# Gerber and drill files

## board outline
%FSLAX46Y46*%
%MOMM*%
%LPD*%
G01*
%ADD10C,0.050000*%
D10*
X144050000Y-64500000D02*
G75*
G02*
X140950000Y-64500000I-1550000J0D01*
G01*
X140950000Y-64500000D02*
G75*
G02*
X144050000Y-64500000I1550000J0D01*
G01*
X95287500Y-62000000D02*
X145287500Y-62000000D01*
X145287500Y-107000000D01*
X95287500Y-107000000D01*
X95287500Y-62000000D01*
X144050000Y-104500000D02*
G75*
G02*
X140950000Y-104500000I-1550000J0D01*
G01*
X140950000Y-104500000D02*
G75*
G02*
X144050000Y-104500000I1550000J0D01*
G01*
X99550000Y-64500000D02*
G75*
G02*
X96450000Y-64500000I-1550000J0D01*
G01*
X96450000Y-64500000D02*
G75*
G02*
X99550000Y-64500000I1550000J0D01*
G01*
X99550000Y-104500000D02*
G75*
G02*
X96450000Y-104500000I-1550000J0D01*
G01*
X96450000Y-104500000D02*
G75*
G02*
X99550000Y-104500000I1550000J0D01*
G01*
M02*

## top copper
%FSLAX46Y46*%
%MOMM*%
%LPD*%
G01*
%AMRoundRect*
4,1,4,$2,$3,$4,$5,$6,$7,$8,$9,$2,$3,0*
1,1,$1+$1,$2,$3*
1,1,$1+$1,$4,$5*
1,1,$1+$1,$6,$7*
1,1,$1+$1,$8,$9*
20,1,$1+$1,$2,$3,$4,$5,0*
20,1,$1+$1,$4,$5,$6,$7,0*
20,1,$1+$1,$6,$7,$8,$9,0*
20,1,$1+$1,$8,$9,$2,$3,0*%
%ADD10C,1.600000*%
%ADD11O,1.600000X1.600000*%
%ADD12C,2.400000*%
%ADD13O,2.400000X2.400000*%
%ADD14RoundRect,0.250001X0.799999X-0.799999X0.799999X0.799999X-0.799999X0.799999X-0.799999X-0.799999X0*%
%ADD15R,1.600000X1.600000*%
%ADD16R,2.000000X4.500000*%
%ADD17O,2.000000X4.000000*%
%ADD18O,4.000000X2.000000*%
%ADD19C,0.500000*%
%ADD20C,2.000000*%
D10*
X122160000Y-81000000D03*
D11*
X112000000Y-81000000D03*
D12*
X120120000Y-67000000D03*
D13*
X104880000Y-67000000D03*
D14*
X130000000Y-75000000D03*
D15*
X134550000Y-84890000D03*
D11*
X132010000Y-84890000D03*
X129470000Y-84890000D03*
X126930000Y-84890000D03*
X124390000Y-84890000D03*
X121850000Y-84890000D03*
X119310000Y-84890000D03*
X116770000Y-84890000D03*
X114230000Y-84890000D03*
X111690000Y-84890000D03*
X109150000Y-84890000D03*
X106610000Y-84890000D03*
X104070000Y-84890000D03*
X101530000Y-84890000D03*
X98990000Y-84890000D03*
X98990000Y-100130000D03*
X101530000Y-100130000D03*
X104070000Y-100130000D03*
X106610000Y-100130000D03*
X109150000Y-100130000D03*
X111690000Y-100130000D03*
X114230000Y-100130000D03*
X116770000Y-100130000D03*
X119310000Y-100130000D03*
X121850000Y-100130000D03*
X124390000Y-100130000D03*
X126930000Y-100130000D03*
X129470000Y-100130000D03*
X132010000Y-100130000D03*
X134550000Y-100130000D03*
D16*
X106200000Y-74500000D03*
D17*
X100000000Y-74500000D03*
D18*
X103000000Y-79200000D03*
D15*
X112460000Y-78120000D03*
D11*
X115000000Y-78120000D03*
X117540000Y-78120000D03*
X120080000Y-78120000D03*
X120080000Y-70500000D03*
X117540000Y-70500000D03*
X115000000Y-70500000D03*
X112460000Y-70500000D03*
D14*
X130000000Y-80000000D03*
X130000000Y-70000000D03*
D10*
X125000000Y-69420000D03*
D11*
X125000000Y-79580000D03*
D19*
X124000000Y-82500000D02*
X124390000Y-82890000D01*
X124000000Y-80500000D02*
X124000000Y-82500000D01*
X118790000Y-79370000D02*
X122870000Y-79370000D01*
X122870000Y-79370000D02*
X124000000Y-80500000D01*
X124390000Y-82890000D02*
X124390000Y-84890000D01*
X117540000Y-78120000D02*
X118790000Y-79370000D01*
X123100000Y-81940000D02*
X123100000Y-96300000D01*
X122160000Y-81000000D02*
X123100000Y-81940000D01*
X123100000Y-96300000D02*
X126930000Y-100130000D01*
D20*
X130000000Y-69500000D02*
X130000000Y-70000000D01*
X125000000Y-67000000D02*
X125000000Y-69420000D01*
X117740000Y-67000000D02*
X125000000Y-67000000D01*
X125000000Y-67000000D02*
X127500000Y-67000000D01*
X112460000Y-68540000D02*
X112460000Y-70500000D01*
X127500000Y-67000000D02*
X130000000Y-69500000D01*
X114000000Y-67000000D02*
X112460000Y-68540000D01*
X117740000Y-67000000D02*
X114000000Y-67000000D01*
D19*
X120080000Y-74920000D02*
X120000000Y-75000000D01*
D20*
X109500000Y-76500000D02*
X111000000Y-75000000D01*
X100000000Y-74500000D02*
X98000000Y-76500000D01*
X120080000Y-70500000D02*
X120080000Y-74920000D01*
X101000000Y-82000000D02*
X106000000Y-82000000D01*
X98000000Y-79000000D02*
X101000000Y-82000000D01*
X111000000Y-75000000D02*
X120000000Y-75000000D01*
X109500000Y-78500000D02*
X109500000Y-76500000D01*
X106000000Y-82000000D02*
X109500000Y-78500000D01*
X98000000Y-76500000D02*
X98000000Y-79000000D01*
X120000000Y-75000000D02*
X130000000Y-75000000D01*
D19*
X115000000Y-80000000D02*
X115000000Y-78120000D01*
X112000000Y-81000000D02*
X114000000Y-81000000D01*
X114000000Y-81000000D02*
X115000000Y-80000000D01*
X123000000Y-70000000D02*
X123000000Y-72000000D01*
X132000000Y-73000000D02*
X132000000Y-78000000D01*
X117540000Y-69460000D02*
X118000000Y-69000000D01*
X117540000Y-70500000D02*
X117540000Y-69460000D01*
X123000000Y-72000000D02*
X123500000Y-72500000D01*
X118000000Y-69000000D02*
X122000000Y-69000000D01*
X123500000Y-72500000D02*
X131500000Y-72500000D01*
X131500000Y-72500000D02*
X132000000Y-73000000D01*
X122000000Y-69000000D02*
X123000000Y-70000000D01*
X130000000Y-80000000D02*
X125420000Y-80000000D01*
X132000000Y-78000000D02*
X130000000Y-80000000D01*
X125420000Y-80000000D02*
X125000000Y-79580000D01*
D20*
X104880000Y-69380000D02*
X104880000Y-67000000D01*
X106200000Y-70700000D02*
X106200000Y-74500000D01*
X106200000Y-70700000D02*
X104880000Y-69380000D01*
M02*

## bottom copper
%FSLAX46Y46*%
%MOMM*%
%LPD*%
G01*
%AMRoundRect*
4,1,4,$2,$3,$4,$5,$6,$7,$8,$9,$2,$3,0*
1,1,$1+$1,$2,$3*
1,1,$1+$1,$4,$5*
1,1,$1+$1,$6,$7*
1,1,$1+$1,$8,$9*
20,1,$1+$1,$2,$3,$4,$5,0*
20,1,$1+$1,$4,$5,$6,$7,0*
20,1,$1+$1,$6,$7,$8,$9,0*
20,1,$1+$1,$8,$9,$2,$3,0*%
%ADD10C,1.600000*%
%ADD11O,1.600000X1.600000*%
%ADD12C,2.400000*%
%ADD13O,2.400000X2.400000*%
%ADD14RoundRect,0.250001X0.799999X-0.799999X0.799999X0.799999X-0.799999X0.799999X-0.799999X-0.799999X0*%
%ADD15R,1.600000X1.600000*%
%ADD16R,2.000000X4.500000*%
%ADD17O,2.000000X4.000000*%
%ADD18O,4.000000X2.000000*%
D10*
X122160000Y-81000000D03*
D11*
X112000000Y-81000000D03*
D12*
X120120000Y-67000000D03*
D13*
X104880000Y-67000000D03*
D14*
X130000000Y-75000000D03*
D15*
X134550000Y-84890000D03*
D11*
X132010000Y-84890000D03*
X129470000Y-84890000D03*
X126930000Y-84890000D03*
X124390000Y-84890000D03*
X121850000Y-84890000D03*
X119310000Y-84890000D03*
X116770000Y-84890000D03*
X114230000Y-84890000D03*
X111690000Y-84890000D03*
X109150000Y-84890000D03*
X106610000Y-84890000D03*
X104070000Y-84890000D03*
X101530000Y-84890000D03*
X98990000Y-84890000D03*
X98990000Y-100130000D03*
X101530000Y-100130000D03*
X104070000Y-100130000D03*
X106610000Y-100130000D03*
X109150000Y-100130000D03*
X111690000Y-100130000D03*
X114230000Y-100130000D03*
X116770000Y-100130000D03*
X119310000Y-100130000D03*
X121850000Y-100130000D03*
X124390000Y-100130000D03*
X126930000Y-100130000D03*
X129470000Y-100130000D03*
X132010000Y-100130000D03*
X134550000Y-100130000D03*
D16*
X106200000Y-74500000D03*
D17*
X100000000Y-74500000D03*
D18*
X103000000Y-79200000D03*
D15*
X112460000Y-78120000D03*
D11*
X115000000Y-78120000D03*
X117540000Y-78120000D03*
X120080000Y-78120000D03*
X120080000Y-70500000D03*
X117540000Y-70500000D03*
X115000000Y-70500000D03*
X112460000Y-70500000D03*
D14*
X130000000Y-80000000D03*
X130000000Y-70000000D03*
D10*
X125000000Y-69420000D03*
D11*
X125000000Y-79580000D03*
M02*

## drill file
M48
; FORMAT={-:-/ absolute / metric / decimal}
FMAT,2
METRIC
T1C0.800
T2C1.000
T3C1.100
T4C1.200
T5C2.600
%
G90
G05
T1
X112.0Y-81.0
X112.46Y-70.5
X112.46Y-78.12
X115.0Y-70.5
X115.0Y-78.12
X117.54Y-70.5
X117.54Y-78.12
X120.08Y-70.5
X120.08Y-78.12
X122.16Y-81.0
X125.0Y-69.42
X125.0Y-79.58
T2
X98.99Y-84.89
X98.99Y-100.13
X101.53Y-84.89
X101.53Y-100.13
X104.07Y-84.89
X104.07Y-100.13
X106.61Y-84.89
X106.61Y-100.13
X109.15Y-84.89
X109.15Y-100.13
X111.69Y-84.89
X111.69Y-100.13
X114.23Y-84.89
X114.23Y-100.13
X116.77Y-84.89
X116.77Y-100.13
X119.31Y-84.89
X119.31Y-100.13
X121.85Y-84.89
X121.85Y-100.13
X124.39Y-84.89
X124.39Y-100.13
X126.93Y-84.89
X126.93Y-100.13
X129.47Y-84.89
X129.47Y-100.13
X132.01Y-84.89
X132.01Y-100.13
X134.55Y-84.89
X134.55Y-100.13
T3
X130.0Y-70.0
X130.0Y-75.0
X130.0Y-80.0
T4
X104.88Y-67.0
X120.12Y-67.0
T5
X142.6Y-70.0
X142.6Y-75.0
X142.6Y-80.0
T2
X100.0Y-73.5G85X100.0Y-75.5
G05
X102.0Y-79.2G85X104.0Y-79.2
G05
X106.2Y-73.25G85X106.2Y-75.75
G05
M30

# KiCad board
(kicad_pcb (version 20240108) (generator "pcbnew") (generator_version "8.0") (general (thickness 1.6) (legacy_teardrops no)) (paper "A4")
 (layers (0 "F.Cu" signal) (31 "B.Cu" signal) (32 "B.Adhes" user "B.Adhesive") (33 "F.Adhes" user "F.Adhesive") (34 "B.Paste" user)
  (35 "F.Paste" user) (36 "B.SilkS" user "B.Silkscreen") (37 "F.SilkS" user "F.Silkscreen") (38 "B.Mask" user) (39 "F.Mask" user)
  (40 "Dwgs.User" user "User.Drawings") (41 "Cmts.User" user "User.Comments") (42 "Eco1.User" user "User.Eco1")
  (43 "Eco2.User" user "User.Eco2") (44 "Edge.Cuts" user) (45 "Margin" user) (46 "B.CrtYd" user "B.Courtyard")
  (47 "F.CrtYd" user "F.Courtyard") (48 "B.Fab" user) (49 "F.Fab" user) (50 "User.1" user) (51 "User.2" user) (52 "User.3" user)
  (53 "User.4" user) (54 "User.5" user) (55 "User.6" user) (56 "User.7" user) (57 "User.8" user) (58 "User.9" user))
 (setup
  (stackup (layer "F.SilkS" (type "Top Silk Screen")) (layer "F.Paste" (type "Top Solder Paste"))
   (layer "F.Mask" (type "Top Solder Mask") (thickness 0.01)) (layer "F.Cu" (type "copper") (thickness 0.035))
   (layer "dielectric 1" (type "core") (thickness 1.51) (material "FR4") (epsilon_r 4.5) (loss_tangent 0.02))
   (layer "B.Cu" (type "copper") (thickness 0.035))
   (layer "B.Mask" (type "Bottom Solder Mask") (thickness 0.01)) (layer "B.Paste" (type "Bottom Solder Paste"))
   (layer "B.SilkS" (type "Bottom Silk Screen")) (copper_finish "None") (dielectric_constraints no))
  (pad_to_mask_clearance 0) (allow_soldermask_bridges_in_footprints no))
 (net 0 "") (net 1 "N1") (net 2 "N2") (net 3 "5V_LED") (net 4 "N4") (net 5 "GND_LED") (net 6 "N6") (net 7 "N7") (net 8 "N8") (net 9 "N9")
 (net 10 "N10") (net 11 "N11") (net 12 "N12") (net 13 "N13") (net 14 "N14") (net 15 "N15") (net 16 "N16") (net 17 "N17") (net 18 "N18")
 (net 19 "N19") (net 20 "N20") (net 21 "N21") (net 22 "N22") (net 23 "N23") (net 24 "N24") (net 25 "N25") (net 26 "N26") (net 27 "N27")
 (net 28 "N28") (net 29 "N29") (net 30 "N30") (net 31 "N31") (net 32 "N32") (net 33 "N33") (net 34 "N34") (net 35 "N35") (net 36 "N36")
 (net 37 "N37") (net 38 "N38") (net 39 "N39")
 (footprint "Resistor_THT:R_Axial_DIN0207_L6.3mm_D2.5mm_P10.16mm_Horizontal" (layer "F.Cu") (at 122.16 81 180)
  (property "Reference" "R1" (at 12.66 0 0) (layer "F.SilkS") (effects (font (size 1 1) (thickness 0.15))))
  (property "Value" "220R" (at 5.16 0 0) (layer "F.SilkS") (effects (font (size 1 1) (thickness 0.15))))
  (pad "1" thru_hole circle (at 0 0 180) (size 1.6 1.6) (drill 0.8) (layers "*.Cu" "*.Mask") (remove_unused_layers no) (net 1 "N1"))
  (pad "2" thru_hole oval (at 10.16 0 180) (size 1.6 1.6) (drill 0.8) (layers "*.Cu" "*.Mask") (remove_unused_layers no) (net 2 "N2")))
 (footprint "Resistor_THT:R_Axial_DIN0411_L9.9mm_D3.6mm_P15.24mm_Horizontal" (layer "F.Cu") (at 120.12 67 180)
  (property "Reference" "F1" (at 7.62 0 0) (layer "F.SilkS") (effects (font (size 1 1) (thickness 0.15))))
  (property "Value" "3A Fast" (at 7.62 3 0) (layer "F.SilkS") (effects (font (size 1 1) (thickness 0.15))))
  (pad "1" thru_hole circle (at 0 0 180) (size 2.4 2.4) (drill 1.2) (layers "*.Cu" "*.Mask") (remove_unused_layers no) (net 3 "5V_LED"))
  (pad "2" thru_hole oval (at 15.24 0 180) (size 2.4 2.4) (drill 1.2) (layers "*.Cu" "*.Mask") (remove_unused_layers no) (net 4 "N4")))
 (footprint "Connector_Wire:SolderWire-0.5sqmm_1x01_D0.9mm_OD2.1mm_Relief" (layer "F.Cu") (at 130 75 90)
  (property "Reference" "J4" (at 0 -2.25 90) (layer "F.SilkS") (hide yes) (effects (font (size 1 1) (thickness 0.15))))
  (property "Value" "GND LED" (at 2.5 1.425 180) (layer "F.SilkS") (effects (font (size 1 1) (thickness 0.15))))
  (pad "" np_thru_hole circle (at 0 12.6 90) (size 2.6 2.6) (drill 2.6) (layers "*.Cu" "*.Mask"))
  (pad "1" thru_hole roundrect (at 0 0 90) (size 2.1 2.1) (drill 1.1) (layers "*.Cu" "*.Mask") (remove_unused_layers no)
   (roundrect_rratio 0.119048) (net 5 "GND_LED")))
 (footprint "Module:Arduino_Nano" (layer "F.Cu") (at 134.55 84.89 -90)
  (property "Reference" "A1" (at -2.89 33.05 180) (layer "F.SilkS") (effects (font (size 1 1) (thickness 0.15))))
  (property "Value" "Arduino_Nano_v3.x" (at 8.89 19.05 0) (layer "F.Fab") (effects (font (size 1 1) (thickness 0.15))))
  (pad "1" thru_hole rect (at 0 0 270) (size 1.6 1.6) (drill 1) (layers "*.Cu" "*.Mask") (remove_unused_layers no) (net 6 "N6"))
  (pad "2" thru_hole oval (at 0 2.54 270) (size 1.6 1.6) (drill 1) (layers "*.Cu" "*.Mask") (remove_unused_layers no) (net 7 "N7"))
  (pad "3" thru_hole oval (at 0 5.08 270) (size 1.6 1.6) (drill 1) (layers "*.Cu" "*.Mask") (remove_unused_layers no) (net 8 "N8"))
  (pad "4" thru_hole oval (at 0 7.62 270) (size 1.6 1.6) (drill 1) (layers "*.Cu" "*.Mask") (remove_unused_layers no) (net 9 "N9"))
  (pad "5" thru_hole oval (at 0 10.16 270) (size 1.6 1.6) (drill 1) (layers "*.Cu" "*.Mask") (remove_unused_layers no) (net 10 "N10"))
  (pad "6" thru_hole oval (at 0 12.7 270) (size 1.6 1.6) (drill 1) (layers "*.Cu" "*.Mask") (remove_unused_layers no) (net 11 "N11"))
  (pad "7" thru_hole oval (at 0 15.24 270) (size 1.6 1.6) (drill 1) (layers "*.Cu" "*.Mask") (remove_unused_layers no) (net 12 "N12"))
  (pad "8" thru_hole oval (at 0 17.78 270) (size 1.6 1.6) (drill 1) (layers "*.Cu" "*.Mask") (remove_unused_layers no) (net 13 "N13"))
  (pad "9" thru_hole oval (at 0 20.32 270) (size 1.6 1.6) (drill 1) (layers "*.Cu" "*.Mask") (remove_unused_layers no) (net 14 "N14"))
  (pad "10" thru_hole oval (at 0 22.86 270) (size 1.6 1.6) (drill 1) (layers "*.Cu" "*.Mask") (remove_unused_layers no) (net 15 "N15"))
  (pad "11" thru_hole oval (at 0 25.4 270) (size 1.6 1.6) (drill 1) (layers "*.Cu" "*.Mask") (remove_unused_layers no) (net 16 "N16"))
  (pad "12" thru_hole oval (at 0 27.94 270) (size 1.6 1.6) (drill 1) (layers "*.Cu" "*.Mask") (remove_unused_layers no) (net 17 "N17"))
  (pad "13" thru_hole oval (at 0 30.48 270) (size 1.6 1.6) (drill 1) (layers "*.Cu" "*.Mask") (remove_unused_layers no) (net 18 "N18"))
  (pad "14" thru_hole oval (at 0 33.02 270) (size 1.6 1.6) (drill 1) (layers "*.Cu" "*.Mask") (remove_unused_layers no) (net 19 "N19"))
  (pad "15" thru_hole oval (at 0 35.56 270) (size 1.6 1.6) (drill 1) (layers "*.Cu" "*.Mask") (remove_unused_layers no) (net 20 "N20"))
  (pad "16" thru_hole oval (at 15.24 35.56 270) (size 1.6 1.6) (drill 1) (layers "*.Cu" "*.Mask") (remove_unused_layers no) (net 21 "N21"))
  (pad "17" thru_hole oval (at 15.24 33.02 270) (size 1.6 1.6) (drill 1) (layers "*.Cu" "*.Mask") (remove_unused_layers no) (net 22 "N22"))
  (pad "18" thru_hole oval (at 15.24 30.48 270) (size 1.6 1.6) (drill 1) (layers "*.Cu" "*.Mask") (remove_unused_layers no) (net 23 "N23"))
  (pad "19" thru_hole oval (at 15.24 27.94 270) (size 1.6 1.6) (drill 1) (layers "*.Cu" "*.Mask") (remove_unused_layers no) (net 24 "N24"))
  (pad "20" thru_hole oval (at 15.24 25.4 270) (size 1.6 1.6) (drill 1) (layers "*.Cu" "*.Mask") (remove_unused_layers no) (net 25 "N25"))
  (pad "21" thru_hole oval (at 15.24 22.86 270) (size 1.6 1.6) (drill 1) (layers "*.Cu" "*.Mask") (remove_unused_layers no) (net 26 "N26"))
  (pad "22" thru_hole oval (at 15.24 20.32 270) (size 1.6 1.6) (drill 1) (layers "*.Cu" "*.Mask") (remove_unused_layers no) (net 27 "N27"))
  (pad "23" thru_hole oval (at 15.24 17.78 270) (size 1.6 1.6) (drill 1) (layers "*.Cu" "*.Mask") (remove_unused_layers no) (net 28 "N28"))
  (pad "24" thru_hole oval (at 15.24 15.24 270) (size 1.6 1.6) (drill 1) (layers "*.Cu" "*.Mask") (remove_unused_layers no) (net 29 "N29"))
  (pad "25" thru_hole oval (at 15.24 12.7 270) (size 1.6 1.6) (drill 1) (layers "*.Cu" "*.Mask") (remove_unused_layers no) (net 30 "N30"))
  (pad "26" thru_hole oval (at 15.24 10.16 270) (size 1.6 1.6) (drill 1) (layers "*.Cu" "*.Mask") (remove_unused_layers no) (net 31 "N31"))
  (pad "27" thru_hole oval (at 15.24 7.62 270) (size 1.6 1.6) (drill 1) (layers "*.Cu" "*.Mask") (remove_unused_layers no) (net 1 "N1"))
  (pad "28" thru_hole oval (at 15.24 5.08 270) (size 1.6 1.6) (drill 1) (layers "*.Cu" "*.Mask") (remove_unused_layers no) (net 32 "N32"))
  (pad "29" thru_hole oval (at 15.24 2.54 270) (size 1.6 1.6) (drill 1) (layers "*.Cu" "*.Mask") (remove_unused_layers no) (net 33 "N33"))
  (pad "30" thru_hole oval (at 15.24 0 270) (size 1.6 1.6) (drill 1) (layers "*.Cu" "*.Mask") (remove_unused_layers no) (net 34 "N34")))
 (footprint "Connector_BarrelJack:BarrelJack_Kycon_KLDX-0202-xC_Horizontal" (layer "F.Cu") (at 106.2 74.5)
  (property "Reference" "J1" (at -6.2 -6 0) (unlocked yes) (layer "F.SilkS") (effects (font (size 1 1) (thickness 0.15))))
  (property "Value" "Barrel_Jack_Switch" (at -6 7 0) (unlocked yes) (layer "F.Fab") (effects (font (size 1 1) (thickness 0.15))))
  (pad "1" thru_hole rect (at 0 0) (size 2 4.5) (drill oval 1 3.5) (layers "*.Cu" "*.Mask") (remove_unused_layers no) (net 4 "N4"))
  (pad "2" thru_hole oval (at -6.2 0) (size 2 4) (drill oval 1 3) (layers "*.Cu" "*.Mask") (remove_unused_layers no) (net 5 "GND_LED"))
  (pad "3" thru_hole oval (at -3.2 4.7 90) (size 2 4) (drill oval 1 3) (layers "*.Cu" "*.Mask") (remove_unused_layers no) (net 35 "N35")))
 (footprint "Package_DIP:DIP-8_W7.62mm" (layer "F.Cu") (at 112.46 78.12 90)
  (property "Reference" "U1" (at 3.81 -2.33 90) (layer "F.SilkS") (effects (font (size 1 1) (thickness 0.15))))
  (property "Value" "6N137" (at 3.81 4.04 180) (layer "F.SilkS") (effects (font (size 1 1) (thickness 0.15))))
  (pad "1" thru_hole rect (at 0 0 90) (size 1.6 1.6) (drill 0.8) (layers "*.Cu" "*.Mask") (remove_unused_layers no) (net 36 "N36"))
  (pad "2" thru_hole oval (at 0 2.54 90) (size 1.6 1.6) (drill 0.8) (layers "*.Cu" "*.Mask") (remove_unused_layers no) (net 2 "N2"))
  (pad "3" thru_hole oval (at 0 5.08 90) (size 1.6 1.6) (drill 0.8) (layers "*.Cu" "*.Mask") (remove_unused_layers no) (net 10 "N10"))
  (pad "4" thru_hole oval (at 0 7.62 90) (size 1.6 1.6) (drill 0.8) (layers "*.Cu" "*.Mask") (remove_unused_layers no) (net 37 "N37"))
  (pad "5" thru_hole oval (at 7.62 7.62 90) (size 1.6 1.6) (drill 0.8) (layers "*.Cu" "*.Mask") (remove_unused_layers no) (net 5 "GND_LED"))
  (pad "6" thru_hole oval (at 7.62 5.08 90) (size 1.6 1.6) (drill 0.8) (layers "*.Cu" "*.Mask") (remove_unused_layers no) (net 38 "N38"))
  (pad "7" thru_hole oval (at 7.62 2.54 90) (size 1.6 1.6) (drill 0.8) (layers "*.Cu" "*.Mask") (remove_unused_layers no) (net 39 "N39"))
  (pad "8" thru_hole oval (at 7.62 0 90) (size 1.6 1.6) (drill 0.8) (layers "*.Cu" "*.Mask") (remove_unused_layers no) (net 3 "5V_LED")))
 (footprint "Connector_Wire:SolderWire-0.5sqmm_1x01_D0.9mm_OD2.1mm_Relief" (layer "F.Cu") (at 130 80 90)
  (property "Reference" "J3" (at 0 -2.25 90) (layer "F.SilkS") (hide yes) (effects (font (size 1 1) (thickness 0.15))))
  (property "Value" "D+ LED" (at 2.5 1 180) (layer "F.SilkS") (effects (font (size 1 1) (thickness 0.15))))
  (pad "" np_thru_hole circle (at 0 12.6 90) (size 2.6 2.6) (drill 2.6) (layers "*.Cu" "*.Mask"))
  (pad "1" thru_hole roundrect (at 0 0 90) (size 2.1 2.1) (drill 1.1) (layers "*.Cu" "*.Mask") (remove_unused_layers no)
   (roundrect_rratio 0.119048) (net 38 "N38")))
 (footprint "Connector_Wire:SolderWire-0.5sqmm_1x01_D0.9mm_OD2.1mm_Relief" (layer "F.Cu") (at 130 70 90)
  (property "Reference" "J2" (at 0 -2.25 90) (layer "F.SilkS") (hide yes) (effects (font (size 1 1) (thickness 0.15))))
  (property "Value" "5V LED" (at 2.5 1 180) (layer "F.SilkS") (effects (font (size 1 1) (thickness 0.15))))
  (pad "" np_thru_hole circle (at 0 12.6 90) (size 2.6 2.6) (drill 2.6) (layers "*.Cu" "*.Mask"))
  (pad "1" thru_hole roundrect (at 0 0 90) (size 2.1 2.1) (drill 1.1) (layers "*.Cu" "*.Mask") (remove_unused_layers no)
   (roundrect_rratio 0.119048) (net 3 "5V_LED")))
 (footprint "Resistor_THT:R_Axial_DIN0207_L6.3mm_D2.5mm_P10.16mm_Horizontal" (layer "F.Cu") (at 125 69.42 -90)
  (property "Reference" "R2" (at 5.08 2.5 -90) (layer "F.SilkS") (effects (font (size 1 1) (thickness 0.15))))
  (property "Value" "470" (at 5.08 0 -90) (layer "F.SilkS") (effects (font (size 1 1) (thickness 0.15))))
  (pad "1" thru_hole circle (at 0 0 270) (size 1.6 1.6) (drill 0.8) (layers "*.Cu" "*.Mask") (remove_unused_layers no) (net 3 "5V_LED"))
  (pad "2" thru_hole oval (at 10.16 0 270) (size 1.6 1.6) (drill 0.8) (layers "*.Cu" "*.Mask") (remove_unused_layers no) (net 38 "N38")))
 (gr_circle (center 142.5 64.5) (end 144.05 64.5) (stroke (width 0.05) (type default)) (fill none) (layer "Edge.Cuts"))
 (gr_rect (start 95.2875 62) (end 145.2875 107) (stroke (width 0.05) (type default)) (fill none) (layer "Edge.Cuts"))
 (gr_circle (center 142.5 104.5) (end 144.05 104.5) (stroke (width 0.05) (type default)) (fill none) (layer "Edge.Cuts"))
 (gr_circle (center 98 64.5) (end 99.55 64.5) (stroke (width 0.05) (type default)) (fill none) (layer "Edge.Cuts"))
 (gr_circle (center 98 104.5) (end 99.55 104.5) (stroke (width 0.05) (type default)) (fill none) (layer "Edge.Cuts"))
 (segment (start 124 82.5) (end 124.39 82.89) (width 0.5) (layer "F.Cu") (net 10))
 (segment (start 124 80.5) (end 124 82.5) (width 0.5) (layer "F.Cu") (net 10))
 (segment (start 118.79 79.37) (end 122.87 79.37) (width 0.5) (layer "F.Cu") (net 10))
 (segment (start 122.87 79.37) (end 124 80.5) (width 0.5) (layer "F.Cu") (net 10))
 (segment (start 124.39 82.89) (end 124.39 84.89) (width 0.5) (layer "F.Cu") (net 10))
 (segment (start 117.54 78.12) (end 118.79 79.37) (width 0.5) (layer "F.Cu") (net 10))
 (segment (start 123.1 81.94) (end 123.1 96.3) (width 0.5) (layer "F.Cu") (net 1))
 (segment (start 122.16 81) (end 123.1 81.94) (width 0.5) (layer "F.Cu") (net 1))
 (segment (start 123.1 96.3) (end 126.93 100.13) (width 0.5) (layer "F.Cu") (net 1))
 (segment (start 130 69.5) (end 130 70) (width 2) (layer "F.Cu") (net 3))
 (segment (start 125 67) (end 125 69.42) (width 2) (layer "F.Cu") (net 3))
 (segment (start 117.74 67) (end 125 67) (width 2) (layer "F.Cu") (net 3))
 (segment (start 125 67) (end 127.5 67) (width 2) (layer "F.Cu") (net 3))
 (segment (start 112.46 68.54) (end 112.46 70.5) (width 2) (layer "F.Cu") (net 3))
 (segment (start 127.5 67) (end 130 69.5) (width 2) (layer "F.Cu") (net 3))
 (segment (start 114 67) (end 112.46 68.54) (width 2) (layer "F.Cu") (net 3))
 (segment (start 117.74 67) (end 114 67) (width 2) (layer "F.Cu") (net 3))
 (segment (start 120.08 74.92) (end 120 75) (width 0.5) (layer "F.Cu") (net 5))
 (segment (start 109.5 76.5) (end 111 75) (width 2) (layer "F.Cu") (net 5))
 (segment (start 100 74.5) (end 98 76.5) (width 2) (layer "F.Cu") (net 5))
 (segment (start 120.08 70.5) (end 120.08 74.92) (width 2) (layer "F.Cu") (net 5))
 (segment (start 101 82) (end 106 82) (width 2) (layer "F.Cu") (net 5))
 (segment (start 98 79) (end 101 82) (width 2) (layer "F.Cu") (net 5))
 (segment (start 111 75) (end 120 75) (width 2) (layer "F.Cu") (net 5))
 (segment (start 109.5 78.5) (end 109.5 76.5) (width 2) (layer "F.Cu") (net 5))
 (segment (start 106 82) (end 109.5 78.5) (width 2) (layer "F.Cu") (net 5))
 (segment (start 98 76.5) (end 98 79) (width 2) (layer "F.Cu") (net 5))
 (segment (start 120 75) (end 130 75) (width 2) (layer "F.Cu") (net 5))
 (segment (start 115 80) (end 115 78.12) (width 0.5) (layer "F.Cu") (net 2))
 (segment (start 112 81) (end 114 81) (width 0.5) (layer "F.Cu") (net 2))
 (segment (start 114 81) (end 115 80) (width 0.5) (layer "F.Cu") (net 2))
 (segment (start 123 70) (end 123 72) (width 0.5) (layer "F.Cu") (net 38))
 (segment (start 132 73) (end 132 78) (width 0.5) (layer "F.Cu") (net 38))
 (segment (start 117.54 69.46) (end 118 69) (width 0.5) (layer "F.Cu") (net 38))
 (segment (start 117.54 70.5) (end 117.54 69.46) (width 0.5) (layer "F.Cu") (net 38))
 (segment (start 123 72) (end 123.5 72.5) (width 0.5) (layer "F.Cu") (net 38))
 (segment (start 118 69) (end 122 69) (width 0.5) (layer "F.Cu") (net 38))
 (segment (start 123.5 72.5) (end 131.5 72.5) (width 0.5) (layer "F.Cu") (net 38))
 (segment (start 131.5 72.5) (end 132 73) (width 0.5) (layer "F.Cu") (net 38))
 (segment (start 122 69) (end 123 70) (width 0.5) (layer "F.Cu") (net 38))
 (segment (start 130 80) (end 125.42 80) (width 0.5) (layer "F.Cu") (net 38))
 (segment (start 132 78) (end 130 80) (width 0.5) (layer "F.Cu") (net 38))
 (segment (start 125.42 80) (end 125 79.58) (width 0.5) (layer "F.Cu") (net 38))
 (segment (start 104.88 69.38) (end 104.88 67) (width 2) (layer "F.Cu") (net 4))
 (segment (start 106.2 70.7) (end 106.2 74.5) (width 2) (layer "F.Cu") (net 4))
 (segment (start 106.2 70.7) (end 104.88 69.38) (width 2) (layer "F.Cu") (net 4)))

